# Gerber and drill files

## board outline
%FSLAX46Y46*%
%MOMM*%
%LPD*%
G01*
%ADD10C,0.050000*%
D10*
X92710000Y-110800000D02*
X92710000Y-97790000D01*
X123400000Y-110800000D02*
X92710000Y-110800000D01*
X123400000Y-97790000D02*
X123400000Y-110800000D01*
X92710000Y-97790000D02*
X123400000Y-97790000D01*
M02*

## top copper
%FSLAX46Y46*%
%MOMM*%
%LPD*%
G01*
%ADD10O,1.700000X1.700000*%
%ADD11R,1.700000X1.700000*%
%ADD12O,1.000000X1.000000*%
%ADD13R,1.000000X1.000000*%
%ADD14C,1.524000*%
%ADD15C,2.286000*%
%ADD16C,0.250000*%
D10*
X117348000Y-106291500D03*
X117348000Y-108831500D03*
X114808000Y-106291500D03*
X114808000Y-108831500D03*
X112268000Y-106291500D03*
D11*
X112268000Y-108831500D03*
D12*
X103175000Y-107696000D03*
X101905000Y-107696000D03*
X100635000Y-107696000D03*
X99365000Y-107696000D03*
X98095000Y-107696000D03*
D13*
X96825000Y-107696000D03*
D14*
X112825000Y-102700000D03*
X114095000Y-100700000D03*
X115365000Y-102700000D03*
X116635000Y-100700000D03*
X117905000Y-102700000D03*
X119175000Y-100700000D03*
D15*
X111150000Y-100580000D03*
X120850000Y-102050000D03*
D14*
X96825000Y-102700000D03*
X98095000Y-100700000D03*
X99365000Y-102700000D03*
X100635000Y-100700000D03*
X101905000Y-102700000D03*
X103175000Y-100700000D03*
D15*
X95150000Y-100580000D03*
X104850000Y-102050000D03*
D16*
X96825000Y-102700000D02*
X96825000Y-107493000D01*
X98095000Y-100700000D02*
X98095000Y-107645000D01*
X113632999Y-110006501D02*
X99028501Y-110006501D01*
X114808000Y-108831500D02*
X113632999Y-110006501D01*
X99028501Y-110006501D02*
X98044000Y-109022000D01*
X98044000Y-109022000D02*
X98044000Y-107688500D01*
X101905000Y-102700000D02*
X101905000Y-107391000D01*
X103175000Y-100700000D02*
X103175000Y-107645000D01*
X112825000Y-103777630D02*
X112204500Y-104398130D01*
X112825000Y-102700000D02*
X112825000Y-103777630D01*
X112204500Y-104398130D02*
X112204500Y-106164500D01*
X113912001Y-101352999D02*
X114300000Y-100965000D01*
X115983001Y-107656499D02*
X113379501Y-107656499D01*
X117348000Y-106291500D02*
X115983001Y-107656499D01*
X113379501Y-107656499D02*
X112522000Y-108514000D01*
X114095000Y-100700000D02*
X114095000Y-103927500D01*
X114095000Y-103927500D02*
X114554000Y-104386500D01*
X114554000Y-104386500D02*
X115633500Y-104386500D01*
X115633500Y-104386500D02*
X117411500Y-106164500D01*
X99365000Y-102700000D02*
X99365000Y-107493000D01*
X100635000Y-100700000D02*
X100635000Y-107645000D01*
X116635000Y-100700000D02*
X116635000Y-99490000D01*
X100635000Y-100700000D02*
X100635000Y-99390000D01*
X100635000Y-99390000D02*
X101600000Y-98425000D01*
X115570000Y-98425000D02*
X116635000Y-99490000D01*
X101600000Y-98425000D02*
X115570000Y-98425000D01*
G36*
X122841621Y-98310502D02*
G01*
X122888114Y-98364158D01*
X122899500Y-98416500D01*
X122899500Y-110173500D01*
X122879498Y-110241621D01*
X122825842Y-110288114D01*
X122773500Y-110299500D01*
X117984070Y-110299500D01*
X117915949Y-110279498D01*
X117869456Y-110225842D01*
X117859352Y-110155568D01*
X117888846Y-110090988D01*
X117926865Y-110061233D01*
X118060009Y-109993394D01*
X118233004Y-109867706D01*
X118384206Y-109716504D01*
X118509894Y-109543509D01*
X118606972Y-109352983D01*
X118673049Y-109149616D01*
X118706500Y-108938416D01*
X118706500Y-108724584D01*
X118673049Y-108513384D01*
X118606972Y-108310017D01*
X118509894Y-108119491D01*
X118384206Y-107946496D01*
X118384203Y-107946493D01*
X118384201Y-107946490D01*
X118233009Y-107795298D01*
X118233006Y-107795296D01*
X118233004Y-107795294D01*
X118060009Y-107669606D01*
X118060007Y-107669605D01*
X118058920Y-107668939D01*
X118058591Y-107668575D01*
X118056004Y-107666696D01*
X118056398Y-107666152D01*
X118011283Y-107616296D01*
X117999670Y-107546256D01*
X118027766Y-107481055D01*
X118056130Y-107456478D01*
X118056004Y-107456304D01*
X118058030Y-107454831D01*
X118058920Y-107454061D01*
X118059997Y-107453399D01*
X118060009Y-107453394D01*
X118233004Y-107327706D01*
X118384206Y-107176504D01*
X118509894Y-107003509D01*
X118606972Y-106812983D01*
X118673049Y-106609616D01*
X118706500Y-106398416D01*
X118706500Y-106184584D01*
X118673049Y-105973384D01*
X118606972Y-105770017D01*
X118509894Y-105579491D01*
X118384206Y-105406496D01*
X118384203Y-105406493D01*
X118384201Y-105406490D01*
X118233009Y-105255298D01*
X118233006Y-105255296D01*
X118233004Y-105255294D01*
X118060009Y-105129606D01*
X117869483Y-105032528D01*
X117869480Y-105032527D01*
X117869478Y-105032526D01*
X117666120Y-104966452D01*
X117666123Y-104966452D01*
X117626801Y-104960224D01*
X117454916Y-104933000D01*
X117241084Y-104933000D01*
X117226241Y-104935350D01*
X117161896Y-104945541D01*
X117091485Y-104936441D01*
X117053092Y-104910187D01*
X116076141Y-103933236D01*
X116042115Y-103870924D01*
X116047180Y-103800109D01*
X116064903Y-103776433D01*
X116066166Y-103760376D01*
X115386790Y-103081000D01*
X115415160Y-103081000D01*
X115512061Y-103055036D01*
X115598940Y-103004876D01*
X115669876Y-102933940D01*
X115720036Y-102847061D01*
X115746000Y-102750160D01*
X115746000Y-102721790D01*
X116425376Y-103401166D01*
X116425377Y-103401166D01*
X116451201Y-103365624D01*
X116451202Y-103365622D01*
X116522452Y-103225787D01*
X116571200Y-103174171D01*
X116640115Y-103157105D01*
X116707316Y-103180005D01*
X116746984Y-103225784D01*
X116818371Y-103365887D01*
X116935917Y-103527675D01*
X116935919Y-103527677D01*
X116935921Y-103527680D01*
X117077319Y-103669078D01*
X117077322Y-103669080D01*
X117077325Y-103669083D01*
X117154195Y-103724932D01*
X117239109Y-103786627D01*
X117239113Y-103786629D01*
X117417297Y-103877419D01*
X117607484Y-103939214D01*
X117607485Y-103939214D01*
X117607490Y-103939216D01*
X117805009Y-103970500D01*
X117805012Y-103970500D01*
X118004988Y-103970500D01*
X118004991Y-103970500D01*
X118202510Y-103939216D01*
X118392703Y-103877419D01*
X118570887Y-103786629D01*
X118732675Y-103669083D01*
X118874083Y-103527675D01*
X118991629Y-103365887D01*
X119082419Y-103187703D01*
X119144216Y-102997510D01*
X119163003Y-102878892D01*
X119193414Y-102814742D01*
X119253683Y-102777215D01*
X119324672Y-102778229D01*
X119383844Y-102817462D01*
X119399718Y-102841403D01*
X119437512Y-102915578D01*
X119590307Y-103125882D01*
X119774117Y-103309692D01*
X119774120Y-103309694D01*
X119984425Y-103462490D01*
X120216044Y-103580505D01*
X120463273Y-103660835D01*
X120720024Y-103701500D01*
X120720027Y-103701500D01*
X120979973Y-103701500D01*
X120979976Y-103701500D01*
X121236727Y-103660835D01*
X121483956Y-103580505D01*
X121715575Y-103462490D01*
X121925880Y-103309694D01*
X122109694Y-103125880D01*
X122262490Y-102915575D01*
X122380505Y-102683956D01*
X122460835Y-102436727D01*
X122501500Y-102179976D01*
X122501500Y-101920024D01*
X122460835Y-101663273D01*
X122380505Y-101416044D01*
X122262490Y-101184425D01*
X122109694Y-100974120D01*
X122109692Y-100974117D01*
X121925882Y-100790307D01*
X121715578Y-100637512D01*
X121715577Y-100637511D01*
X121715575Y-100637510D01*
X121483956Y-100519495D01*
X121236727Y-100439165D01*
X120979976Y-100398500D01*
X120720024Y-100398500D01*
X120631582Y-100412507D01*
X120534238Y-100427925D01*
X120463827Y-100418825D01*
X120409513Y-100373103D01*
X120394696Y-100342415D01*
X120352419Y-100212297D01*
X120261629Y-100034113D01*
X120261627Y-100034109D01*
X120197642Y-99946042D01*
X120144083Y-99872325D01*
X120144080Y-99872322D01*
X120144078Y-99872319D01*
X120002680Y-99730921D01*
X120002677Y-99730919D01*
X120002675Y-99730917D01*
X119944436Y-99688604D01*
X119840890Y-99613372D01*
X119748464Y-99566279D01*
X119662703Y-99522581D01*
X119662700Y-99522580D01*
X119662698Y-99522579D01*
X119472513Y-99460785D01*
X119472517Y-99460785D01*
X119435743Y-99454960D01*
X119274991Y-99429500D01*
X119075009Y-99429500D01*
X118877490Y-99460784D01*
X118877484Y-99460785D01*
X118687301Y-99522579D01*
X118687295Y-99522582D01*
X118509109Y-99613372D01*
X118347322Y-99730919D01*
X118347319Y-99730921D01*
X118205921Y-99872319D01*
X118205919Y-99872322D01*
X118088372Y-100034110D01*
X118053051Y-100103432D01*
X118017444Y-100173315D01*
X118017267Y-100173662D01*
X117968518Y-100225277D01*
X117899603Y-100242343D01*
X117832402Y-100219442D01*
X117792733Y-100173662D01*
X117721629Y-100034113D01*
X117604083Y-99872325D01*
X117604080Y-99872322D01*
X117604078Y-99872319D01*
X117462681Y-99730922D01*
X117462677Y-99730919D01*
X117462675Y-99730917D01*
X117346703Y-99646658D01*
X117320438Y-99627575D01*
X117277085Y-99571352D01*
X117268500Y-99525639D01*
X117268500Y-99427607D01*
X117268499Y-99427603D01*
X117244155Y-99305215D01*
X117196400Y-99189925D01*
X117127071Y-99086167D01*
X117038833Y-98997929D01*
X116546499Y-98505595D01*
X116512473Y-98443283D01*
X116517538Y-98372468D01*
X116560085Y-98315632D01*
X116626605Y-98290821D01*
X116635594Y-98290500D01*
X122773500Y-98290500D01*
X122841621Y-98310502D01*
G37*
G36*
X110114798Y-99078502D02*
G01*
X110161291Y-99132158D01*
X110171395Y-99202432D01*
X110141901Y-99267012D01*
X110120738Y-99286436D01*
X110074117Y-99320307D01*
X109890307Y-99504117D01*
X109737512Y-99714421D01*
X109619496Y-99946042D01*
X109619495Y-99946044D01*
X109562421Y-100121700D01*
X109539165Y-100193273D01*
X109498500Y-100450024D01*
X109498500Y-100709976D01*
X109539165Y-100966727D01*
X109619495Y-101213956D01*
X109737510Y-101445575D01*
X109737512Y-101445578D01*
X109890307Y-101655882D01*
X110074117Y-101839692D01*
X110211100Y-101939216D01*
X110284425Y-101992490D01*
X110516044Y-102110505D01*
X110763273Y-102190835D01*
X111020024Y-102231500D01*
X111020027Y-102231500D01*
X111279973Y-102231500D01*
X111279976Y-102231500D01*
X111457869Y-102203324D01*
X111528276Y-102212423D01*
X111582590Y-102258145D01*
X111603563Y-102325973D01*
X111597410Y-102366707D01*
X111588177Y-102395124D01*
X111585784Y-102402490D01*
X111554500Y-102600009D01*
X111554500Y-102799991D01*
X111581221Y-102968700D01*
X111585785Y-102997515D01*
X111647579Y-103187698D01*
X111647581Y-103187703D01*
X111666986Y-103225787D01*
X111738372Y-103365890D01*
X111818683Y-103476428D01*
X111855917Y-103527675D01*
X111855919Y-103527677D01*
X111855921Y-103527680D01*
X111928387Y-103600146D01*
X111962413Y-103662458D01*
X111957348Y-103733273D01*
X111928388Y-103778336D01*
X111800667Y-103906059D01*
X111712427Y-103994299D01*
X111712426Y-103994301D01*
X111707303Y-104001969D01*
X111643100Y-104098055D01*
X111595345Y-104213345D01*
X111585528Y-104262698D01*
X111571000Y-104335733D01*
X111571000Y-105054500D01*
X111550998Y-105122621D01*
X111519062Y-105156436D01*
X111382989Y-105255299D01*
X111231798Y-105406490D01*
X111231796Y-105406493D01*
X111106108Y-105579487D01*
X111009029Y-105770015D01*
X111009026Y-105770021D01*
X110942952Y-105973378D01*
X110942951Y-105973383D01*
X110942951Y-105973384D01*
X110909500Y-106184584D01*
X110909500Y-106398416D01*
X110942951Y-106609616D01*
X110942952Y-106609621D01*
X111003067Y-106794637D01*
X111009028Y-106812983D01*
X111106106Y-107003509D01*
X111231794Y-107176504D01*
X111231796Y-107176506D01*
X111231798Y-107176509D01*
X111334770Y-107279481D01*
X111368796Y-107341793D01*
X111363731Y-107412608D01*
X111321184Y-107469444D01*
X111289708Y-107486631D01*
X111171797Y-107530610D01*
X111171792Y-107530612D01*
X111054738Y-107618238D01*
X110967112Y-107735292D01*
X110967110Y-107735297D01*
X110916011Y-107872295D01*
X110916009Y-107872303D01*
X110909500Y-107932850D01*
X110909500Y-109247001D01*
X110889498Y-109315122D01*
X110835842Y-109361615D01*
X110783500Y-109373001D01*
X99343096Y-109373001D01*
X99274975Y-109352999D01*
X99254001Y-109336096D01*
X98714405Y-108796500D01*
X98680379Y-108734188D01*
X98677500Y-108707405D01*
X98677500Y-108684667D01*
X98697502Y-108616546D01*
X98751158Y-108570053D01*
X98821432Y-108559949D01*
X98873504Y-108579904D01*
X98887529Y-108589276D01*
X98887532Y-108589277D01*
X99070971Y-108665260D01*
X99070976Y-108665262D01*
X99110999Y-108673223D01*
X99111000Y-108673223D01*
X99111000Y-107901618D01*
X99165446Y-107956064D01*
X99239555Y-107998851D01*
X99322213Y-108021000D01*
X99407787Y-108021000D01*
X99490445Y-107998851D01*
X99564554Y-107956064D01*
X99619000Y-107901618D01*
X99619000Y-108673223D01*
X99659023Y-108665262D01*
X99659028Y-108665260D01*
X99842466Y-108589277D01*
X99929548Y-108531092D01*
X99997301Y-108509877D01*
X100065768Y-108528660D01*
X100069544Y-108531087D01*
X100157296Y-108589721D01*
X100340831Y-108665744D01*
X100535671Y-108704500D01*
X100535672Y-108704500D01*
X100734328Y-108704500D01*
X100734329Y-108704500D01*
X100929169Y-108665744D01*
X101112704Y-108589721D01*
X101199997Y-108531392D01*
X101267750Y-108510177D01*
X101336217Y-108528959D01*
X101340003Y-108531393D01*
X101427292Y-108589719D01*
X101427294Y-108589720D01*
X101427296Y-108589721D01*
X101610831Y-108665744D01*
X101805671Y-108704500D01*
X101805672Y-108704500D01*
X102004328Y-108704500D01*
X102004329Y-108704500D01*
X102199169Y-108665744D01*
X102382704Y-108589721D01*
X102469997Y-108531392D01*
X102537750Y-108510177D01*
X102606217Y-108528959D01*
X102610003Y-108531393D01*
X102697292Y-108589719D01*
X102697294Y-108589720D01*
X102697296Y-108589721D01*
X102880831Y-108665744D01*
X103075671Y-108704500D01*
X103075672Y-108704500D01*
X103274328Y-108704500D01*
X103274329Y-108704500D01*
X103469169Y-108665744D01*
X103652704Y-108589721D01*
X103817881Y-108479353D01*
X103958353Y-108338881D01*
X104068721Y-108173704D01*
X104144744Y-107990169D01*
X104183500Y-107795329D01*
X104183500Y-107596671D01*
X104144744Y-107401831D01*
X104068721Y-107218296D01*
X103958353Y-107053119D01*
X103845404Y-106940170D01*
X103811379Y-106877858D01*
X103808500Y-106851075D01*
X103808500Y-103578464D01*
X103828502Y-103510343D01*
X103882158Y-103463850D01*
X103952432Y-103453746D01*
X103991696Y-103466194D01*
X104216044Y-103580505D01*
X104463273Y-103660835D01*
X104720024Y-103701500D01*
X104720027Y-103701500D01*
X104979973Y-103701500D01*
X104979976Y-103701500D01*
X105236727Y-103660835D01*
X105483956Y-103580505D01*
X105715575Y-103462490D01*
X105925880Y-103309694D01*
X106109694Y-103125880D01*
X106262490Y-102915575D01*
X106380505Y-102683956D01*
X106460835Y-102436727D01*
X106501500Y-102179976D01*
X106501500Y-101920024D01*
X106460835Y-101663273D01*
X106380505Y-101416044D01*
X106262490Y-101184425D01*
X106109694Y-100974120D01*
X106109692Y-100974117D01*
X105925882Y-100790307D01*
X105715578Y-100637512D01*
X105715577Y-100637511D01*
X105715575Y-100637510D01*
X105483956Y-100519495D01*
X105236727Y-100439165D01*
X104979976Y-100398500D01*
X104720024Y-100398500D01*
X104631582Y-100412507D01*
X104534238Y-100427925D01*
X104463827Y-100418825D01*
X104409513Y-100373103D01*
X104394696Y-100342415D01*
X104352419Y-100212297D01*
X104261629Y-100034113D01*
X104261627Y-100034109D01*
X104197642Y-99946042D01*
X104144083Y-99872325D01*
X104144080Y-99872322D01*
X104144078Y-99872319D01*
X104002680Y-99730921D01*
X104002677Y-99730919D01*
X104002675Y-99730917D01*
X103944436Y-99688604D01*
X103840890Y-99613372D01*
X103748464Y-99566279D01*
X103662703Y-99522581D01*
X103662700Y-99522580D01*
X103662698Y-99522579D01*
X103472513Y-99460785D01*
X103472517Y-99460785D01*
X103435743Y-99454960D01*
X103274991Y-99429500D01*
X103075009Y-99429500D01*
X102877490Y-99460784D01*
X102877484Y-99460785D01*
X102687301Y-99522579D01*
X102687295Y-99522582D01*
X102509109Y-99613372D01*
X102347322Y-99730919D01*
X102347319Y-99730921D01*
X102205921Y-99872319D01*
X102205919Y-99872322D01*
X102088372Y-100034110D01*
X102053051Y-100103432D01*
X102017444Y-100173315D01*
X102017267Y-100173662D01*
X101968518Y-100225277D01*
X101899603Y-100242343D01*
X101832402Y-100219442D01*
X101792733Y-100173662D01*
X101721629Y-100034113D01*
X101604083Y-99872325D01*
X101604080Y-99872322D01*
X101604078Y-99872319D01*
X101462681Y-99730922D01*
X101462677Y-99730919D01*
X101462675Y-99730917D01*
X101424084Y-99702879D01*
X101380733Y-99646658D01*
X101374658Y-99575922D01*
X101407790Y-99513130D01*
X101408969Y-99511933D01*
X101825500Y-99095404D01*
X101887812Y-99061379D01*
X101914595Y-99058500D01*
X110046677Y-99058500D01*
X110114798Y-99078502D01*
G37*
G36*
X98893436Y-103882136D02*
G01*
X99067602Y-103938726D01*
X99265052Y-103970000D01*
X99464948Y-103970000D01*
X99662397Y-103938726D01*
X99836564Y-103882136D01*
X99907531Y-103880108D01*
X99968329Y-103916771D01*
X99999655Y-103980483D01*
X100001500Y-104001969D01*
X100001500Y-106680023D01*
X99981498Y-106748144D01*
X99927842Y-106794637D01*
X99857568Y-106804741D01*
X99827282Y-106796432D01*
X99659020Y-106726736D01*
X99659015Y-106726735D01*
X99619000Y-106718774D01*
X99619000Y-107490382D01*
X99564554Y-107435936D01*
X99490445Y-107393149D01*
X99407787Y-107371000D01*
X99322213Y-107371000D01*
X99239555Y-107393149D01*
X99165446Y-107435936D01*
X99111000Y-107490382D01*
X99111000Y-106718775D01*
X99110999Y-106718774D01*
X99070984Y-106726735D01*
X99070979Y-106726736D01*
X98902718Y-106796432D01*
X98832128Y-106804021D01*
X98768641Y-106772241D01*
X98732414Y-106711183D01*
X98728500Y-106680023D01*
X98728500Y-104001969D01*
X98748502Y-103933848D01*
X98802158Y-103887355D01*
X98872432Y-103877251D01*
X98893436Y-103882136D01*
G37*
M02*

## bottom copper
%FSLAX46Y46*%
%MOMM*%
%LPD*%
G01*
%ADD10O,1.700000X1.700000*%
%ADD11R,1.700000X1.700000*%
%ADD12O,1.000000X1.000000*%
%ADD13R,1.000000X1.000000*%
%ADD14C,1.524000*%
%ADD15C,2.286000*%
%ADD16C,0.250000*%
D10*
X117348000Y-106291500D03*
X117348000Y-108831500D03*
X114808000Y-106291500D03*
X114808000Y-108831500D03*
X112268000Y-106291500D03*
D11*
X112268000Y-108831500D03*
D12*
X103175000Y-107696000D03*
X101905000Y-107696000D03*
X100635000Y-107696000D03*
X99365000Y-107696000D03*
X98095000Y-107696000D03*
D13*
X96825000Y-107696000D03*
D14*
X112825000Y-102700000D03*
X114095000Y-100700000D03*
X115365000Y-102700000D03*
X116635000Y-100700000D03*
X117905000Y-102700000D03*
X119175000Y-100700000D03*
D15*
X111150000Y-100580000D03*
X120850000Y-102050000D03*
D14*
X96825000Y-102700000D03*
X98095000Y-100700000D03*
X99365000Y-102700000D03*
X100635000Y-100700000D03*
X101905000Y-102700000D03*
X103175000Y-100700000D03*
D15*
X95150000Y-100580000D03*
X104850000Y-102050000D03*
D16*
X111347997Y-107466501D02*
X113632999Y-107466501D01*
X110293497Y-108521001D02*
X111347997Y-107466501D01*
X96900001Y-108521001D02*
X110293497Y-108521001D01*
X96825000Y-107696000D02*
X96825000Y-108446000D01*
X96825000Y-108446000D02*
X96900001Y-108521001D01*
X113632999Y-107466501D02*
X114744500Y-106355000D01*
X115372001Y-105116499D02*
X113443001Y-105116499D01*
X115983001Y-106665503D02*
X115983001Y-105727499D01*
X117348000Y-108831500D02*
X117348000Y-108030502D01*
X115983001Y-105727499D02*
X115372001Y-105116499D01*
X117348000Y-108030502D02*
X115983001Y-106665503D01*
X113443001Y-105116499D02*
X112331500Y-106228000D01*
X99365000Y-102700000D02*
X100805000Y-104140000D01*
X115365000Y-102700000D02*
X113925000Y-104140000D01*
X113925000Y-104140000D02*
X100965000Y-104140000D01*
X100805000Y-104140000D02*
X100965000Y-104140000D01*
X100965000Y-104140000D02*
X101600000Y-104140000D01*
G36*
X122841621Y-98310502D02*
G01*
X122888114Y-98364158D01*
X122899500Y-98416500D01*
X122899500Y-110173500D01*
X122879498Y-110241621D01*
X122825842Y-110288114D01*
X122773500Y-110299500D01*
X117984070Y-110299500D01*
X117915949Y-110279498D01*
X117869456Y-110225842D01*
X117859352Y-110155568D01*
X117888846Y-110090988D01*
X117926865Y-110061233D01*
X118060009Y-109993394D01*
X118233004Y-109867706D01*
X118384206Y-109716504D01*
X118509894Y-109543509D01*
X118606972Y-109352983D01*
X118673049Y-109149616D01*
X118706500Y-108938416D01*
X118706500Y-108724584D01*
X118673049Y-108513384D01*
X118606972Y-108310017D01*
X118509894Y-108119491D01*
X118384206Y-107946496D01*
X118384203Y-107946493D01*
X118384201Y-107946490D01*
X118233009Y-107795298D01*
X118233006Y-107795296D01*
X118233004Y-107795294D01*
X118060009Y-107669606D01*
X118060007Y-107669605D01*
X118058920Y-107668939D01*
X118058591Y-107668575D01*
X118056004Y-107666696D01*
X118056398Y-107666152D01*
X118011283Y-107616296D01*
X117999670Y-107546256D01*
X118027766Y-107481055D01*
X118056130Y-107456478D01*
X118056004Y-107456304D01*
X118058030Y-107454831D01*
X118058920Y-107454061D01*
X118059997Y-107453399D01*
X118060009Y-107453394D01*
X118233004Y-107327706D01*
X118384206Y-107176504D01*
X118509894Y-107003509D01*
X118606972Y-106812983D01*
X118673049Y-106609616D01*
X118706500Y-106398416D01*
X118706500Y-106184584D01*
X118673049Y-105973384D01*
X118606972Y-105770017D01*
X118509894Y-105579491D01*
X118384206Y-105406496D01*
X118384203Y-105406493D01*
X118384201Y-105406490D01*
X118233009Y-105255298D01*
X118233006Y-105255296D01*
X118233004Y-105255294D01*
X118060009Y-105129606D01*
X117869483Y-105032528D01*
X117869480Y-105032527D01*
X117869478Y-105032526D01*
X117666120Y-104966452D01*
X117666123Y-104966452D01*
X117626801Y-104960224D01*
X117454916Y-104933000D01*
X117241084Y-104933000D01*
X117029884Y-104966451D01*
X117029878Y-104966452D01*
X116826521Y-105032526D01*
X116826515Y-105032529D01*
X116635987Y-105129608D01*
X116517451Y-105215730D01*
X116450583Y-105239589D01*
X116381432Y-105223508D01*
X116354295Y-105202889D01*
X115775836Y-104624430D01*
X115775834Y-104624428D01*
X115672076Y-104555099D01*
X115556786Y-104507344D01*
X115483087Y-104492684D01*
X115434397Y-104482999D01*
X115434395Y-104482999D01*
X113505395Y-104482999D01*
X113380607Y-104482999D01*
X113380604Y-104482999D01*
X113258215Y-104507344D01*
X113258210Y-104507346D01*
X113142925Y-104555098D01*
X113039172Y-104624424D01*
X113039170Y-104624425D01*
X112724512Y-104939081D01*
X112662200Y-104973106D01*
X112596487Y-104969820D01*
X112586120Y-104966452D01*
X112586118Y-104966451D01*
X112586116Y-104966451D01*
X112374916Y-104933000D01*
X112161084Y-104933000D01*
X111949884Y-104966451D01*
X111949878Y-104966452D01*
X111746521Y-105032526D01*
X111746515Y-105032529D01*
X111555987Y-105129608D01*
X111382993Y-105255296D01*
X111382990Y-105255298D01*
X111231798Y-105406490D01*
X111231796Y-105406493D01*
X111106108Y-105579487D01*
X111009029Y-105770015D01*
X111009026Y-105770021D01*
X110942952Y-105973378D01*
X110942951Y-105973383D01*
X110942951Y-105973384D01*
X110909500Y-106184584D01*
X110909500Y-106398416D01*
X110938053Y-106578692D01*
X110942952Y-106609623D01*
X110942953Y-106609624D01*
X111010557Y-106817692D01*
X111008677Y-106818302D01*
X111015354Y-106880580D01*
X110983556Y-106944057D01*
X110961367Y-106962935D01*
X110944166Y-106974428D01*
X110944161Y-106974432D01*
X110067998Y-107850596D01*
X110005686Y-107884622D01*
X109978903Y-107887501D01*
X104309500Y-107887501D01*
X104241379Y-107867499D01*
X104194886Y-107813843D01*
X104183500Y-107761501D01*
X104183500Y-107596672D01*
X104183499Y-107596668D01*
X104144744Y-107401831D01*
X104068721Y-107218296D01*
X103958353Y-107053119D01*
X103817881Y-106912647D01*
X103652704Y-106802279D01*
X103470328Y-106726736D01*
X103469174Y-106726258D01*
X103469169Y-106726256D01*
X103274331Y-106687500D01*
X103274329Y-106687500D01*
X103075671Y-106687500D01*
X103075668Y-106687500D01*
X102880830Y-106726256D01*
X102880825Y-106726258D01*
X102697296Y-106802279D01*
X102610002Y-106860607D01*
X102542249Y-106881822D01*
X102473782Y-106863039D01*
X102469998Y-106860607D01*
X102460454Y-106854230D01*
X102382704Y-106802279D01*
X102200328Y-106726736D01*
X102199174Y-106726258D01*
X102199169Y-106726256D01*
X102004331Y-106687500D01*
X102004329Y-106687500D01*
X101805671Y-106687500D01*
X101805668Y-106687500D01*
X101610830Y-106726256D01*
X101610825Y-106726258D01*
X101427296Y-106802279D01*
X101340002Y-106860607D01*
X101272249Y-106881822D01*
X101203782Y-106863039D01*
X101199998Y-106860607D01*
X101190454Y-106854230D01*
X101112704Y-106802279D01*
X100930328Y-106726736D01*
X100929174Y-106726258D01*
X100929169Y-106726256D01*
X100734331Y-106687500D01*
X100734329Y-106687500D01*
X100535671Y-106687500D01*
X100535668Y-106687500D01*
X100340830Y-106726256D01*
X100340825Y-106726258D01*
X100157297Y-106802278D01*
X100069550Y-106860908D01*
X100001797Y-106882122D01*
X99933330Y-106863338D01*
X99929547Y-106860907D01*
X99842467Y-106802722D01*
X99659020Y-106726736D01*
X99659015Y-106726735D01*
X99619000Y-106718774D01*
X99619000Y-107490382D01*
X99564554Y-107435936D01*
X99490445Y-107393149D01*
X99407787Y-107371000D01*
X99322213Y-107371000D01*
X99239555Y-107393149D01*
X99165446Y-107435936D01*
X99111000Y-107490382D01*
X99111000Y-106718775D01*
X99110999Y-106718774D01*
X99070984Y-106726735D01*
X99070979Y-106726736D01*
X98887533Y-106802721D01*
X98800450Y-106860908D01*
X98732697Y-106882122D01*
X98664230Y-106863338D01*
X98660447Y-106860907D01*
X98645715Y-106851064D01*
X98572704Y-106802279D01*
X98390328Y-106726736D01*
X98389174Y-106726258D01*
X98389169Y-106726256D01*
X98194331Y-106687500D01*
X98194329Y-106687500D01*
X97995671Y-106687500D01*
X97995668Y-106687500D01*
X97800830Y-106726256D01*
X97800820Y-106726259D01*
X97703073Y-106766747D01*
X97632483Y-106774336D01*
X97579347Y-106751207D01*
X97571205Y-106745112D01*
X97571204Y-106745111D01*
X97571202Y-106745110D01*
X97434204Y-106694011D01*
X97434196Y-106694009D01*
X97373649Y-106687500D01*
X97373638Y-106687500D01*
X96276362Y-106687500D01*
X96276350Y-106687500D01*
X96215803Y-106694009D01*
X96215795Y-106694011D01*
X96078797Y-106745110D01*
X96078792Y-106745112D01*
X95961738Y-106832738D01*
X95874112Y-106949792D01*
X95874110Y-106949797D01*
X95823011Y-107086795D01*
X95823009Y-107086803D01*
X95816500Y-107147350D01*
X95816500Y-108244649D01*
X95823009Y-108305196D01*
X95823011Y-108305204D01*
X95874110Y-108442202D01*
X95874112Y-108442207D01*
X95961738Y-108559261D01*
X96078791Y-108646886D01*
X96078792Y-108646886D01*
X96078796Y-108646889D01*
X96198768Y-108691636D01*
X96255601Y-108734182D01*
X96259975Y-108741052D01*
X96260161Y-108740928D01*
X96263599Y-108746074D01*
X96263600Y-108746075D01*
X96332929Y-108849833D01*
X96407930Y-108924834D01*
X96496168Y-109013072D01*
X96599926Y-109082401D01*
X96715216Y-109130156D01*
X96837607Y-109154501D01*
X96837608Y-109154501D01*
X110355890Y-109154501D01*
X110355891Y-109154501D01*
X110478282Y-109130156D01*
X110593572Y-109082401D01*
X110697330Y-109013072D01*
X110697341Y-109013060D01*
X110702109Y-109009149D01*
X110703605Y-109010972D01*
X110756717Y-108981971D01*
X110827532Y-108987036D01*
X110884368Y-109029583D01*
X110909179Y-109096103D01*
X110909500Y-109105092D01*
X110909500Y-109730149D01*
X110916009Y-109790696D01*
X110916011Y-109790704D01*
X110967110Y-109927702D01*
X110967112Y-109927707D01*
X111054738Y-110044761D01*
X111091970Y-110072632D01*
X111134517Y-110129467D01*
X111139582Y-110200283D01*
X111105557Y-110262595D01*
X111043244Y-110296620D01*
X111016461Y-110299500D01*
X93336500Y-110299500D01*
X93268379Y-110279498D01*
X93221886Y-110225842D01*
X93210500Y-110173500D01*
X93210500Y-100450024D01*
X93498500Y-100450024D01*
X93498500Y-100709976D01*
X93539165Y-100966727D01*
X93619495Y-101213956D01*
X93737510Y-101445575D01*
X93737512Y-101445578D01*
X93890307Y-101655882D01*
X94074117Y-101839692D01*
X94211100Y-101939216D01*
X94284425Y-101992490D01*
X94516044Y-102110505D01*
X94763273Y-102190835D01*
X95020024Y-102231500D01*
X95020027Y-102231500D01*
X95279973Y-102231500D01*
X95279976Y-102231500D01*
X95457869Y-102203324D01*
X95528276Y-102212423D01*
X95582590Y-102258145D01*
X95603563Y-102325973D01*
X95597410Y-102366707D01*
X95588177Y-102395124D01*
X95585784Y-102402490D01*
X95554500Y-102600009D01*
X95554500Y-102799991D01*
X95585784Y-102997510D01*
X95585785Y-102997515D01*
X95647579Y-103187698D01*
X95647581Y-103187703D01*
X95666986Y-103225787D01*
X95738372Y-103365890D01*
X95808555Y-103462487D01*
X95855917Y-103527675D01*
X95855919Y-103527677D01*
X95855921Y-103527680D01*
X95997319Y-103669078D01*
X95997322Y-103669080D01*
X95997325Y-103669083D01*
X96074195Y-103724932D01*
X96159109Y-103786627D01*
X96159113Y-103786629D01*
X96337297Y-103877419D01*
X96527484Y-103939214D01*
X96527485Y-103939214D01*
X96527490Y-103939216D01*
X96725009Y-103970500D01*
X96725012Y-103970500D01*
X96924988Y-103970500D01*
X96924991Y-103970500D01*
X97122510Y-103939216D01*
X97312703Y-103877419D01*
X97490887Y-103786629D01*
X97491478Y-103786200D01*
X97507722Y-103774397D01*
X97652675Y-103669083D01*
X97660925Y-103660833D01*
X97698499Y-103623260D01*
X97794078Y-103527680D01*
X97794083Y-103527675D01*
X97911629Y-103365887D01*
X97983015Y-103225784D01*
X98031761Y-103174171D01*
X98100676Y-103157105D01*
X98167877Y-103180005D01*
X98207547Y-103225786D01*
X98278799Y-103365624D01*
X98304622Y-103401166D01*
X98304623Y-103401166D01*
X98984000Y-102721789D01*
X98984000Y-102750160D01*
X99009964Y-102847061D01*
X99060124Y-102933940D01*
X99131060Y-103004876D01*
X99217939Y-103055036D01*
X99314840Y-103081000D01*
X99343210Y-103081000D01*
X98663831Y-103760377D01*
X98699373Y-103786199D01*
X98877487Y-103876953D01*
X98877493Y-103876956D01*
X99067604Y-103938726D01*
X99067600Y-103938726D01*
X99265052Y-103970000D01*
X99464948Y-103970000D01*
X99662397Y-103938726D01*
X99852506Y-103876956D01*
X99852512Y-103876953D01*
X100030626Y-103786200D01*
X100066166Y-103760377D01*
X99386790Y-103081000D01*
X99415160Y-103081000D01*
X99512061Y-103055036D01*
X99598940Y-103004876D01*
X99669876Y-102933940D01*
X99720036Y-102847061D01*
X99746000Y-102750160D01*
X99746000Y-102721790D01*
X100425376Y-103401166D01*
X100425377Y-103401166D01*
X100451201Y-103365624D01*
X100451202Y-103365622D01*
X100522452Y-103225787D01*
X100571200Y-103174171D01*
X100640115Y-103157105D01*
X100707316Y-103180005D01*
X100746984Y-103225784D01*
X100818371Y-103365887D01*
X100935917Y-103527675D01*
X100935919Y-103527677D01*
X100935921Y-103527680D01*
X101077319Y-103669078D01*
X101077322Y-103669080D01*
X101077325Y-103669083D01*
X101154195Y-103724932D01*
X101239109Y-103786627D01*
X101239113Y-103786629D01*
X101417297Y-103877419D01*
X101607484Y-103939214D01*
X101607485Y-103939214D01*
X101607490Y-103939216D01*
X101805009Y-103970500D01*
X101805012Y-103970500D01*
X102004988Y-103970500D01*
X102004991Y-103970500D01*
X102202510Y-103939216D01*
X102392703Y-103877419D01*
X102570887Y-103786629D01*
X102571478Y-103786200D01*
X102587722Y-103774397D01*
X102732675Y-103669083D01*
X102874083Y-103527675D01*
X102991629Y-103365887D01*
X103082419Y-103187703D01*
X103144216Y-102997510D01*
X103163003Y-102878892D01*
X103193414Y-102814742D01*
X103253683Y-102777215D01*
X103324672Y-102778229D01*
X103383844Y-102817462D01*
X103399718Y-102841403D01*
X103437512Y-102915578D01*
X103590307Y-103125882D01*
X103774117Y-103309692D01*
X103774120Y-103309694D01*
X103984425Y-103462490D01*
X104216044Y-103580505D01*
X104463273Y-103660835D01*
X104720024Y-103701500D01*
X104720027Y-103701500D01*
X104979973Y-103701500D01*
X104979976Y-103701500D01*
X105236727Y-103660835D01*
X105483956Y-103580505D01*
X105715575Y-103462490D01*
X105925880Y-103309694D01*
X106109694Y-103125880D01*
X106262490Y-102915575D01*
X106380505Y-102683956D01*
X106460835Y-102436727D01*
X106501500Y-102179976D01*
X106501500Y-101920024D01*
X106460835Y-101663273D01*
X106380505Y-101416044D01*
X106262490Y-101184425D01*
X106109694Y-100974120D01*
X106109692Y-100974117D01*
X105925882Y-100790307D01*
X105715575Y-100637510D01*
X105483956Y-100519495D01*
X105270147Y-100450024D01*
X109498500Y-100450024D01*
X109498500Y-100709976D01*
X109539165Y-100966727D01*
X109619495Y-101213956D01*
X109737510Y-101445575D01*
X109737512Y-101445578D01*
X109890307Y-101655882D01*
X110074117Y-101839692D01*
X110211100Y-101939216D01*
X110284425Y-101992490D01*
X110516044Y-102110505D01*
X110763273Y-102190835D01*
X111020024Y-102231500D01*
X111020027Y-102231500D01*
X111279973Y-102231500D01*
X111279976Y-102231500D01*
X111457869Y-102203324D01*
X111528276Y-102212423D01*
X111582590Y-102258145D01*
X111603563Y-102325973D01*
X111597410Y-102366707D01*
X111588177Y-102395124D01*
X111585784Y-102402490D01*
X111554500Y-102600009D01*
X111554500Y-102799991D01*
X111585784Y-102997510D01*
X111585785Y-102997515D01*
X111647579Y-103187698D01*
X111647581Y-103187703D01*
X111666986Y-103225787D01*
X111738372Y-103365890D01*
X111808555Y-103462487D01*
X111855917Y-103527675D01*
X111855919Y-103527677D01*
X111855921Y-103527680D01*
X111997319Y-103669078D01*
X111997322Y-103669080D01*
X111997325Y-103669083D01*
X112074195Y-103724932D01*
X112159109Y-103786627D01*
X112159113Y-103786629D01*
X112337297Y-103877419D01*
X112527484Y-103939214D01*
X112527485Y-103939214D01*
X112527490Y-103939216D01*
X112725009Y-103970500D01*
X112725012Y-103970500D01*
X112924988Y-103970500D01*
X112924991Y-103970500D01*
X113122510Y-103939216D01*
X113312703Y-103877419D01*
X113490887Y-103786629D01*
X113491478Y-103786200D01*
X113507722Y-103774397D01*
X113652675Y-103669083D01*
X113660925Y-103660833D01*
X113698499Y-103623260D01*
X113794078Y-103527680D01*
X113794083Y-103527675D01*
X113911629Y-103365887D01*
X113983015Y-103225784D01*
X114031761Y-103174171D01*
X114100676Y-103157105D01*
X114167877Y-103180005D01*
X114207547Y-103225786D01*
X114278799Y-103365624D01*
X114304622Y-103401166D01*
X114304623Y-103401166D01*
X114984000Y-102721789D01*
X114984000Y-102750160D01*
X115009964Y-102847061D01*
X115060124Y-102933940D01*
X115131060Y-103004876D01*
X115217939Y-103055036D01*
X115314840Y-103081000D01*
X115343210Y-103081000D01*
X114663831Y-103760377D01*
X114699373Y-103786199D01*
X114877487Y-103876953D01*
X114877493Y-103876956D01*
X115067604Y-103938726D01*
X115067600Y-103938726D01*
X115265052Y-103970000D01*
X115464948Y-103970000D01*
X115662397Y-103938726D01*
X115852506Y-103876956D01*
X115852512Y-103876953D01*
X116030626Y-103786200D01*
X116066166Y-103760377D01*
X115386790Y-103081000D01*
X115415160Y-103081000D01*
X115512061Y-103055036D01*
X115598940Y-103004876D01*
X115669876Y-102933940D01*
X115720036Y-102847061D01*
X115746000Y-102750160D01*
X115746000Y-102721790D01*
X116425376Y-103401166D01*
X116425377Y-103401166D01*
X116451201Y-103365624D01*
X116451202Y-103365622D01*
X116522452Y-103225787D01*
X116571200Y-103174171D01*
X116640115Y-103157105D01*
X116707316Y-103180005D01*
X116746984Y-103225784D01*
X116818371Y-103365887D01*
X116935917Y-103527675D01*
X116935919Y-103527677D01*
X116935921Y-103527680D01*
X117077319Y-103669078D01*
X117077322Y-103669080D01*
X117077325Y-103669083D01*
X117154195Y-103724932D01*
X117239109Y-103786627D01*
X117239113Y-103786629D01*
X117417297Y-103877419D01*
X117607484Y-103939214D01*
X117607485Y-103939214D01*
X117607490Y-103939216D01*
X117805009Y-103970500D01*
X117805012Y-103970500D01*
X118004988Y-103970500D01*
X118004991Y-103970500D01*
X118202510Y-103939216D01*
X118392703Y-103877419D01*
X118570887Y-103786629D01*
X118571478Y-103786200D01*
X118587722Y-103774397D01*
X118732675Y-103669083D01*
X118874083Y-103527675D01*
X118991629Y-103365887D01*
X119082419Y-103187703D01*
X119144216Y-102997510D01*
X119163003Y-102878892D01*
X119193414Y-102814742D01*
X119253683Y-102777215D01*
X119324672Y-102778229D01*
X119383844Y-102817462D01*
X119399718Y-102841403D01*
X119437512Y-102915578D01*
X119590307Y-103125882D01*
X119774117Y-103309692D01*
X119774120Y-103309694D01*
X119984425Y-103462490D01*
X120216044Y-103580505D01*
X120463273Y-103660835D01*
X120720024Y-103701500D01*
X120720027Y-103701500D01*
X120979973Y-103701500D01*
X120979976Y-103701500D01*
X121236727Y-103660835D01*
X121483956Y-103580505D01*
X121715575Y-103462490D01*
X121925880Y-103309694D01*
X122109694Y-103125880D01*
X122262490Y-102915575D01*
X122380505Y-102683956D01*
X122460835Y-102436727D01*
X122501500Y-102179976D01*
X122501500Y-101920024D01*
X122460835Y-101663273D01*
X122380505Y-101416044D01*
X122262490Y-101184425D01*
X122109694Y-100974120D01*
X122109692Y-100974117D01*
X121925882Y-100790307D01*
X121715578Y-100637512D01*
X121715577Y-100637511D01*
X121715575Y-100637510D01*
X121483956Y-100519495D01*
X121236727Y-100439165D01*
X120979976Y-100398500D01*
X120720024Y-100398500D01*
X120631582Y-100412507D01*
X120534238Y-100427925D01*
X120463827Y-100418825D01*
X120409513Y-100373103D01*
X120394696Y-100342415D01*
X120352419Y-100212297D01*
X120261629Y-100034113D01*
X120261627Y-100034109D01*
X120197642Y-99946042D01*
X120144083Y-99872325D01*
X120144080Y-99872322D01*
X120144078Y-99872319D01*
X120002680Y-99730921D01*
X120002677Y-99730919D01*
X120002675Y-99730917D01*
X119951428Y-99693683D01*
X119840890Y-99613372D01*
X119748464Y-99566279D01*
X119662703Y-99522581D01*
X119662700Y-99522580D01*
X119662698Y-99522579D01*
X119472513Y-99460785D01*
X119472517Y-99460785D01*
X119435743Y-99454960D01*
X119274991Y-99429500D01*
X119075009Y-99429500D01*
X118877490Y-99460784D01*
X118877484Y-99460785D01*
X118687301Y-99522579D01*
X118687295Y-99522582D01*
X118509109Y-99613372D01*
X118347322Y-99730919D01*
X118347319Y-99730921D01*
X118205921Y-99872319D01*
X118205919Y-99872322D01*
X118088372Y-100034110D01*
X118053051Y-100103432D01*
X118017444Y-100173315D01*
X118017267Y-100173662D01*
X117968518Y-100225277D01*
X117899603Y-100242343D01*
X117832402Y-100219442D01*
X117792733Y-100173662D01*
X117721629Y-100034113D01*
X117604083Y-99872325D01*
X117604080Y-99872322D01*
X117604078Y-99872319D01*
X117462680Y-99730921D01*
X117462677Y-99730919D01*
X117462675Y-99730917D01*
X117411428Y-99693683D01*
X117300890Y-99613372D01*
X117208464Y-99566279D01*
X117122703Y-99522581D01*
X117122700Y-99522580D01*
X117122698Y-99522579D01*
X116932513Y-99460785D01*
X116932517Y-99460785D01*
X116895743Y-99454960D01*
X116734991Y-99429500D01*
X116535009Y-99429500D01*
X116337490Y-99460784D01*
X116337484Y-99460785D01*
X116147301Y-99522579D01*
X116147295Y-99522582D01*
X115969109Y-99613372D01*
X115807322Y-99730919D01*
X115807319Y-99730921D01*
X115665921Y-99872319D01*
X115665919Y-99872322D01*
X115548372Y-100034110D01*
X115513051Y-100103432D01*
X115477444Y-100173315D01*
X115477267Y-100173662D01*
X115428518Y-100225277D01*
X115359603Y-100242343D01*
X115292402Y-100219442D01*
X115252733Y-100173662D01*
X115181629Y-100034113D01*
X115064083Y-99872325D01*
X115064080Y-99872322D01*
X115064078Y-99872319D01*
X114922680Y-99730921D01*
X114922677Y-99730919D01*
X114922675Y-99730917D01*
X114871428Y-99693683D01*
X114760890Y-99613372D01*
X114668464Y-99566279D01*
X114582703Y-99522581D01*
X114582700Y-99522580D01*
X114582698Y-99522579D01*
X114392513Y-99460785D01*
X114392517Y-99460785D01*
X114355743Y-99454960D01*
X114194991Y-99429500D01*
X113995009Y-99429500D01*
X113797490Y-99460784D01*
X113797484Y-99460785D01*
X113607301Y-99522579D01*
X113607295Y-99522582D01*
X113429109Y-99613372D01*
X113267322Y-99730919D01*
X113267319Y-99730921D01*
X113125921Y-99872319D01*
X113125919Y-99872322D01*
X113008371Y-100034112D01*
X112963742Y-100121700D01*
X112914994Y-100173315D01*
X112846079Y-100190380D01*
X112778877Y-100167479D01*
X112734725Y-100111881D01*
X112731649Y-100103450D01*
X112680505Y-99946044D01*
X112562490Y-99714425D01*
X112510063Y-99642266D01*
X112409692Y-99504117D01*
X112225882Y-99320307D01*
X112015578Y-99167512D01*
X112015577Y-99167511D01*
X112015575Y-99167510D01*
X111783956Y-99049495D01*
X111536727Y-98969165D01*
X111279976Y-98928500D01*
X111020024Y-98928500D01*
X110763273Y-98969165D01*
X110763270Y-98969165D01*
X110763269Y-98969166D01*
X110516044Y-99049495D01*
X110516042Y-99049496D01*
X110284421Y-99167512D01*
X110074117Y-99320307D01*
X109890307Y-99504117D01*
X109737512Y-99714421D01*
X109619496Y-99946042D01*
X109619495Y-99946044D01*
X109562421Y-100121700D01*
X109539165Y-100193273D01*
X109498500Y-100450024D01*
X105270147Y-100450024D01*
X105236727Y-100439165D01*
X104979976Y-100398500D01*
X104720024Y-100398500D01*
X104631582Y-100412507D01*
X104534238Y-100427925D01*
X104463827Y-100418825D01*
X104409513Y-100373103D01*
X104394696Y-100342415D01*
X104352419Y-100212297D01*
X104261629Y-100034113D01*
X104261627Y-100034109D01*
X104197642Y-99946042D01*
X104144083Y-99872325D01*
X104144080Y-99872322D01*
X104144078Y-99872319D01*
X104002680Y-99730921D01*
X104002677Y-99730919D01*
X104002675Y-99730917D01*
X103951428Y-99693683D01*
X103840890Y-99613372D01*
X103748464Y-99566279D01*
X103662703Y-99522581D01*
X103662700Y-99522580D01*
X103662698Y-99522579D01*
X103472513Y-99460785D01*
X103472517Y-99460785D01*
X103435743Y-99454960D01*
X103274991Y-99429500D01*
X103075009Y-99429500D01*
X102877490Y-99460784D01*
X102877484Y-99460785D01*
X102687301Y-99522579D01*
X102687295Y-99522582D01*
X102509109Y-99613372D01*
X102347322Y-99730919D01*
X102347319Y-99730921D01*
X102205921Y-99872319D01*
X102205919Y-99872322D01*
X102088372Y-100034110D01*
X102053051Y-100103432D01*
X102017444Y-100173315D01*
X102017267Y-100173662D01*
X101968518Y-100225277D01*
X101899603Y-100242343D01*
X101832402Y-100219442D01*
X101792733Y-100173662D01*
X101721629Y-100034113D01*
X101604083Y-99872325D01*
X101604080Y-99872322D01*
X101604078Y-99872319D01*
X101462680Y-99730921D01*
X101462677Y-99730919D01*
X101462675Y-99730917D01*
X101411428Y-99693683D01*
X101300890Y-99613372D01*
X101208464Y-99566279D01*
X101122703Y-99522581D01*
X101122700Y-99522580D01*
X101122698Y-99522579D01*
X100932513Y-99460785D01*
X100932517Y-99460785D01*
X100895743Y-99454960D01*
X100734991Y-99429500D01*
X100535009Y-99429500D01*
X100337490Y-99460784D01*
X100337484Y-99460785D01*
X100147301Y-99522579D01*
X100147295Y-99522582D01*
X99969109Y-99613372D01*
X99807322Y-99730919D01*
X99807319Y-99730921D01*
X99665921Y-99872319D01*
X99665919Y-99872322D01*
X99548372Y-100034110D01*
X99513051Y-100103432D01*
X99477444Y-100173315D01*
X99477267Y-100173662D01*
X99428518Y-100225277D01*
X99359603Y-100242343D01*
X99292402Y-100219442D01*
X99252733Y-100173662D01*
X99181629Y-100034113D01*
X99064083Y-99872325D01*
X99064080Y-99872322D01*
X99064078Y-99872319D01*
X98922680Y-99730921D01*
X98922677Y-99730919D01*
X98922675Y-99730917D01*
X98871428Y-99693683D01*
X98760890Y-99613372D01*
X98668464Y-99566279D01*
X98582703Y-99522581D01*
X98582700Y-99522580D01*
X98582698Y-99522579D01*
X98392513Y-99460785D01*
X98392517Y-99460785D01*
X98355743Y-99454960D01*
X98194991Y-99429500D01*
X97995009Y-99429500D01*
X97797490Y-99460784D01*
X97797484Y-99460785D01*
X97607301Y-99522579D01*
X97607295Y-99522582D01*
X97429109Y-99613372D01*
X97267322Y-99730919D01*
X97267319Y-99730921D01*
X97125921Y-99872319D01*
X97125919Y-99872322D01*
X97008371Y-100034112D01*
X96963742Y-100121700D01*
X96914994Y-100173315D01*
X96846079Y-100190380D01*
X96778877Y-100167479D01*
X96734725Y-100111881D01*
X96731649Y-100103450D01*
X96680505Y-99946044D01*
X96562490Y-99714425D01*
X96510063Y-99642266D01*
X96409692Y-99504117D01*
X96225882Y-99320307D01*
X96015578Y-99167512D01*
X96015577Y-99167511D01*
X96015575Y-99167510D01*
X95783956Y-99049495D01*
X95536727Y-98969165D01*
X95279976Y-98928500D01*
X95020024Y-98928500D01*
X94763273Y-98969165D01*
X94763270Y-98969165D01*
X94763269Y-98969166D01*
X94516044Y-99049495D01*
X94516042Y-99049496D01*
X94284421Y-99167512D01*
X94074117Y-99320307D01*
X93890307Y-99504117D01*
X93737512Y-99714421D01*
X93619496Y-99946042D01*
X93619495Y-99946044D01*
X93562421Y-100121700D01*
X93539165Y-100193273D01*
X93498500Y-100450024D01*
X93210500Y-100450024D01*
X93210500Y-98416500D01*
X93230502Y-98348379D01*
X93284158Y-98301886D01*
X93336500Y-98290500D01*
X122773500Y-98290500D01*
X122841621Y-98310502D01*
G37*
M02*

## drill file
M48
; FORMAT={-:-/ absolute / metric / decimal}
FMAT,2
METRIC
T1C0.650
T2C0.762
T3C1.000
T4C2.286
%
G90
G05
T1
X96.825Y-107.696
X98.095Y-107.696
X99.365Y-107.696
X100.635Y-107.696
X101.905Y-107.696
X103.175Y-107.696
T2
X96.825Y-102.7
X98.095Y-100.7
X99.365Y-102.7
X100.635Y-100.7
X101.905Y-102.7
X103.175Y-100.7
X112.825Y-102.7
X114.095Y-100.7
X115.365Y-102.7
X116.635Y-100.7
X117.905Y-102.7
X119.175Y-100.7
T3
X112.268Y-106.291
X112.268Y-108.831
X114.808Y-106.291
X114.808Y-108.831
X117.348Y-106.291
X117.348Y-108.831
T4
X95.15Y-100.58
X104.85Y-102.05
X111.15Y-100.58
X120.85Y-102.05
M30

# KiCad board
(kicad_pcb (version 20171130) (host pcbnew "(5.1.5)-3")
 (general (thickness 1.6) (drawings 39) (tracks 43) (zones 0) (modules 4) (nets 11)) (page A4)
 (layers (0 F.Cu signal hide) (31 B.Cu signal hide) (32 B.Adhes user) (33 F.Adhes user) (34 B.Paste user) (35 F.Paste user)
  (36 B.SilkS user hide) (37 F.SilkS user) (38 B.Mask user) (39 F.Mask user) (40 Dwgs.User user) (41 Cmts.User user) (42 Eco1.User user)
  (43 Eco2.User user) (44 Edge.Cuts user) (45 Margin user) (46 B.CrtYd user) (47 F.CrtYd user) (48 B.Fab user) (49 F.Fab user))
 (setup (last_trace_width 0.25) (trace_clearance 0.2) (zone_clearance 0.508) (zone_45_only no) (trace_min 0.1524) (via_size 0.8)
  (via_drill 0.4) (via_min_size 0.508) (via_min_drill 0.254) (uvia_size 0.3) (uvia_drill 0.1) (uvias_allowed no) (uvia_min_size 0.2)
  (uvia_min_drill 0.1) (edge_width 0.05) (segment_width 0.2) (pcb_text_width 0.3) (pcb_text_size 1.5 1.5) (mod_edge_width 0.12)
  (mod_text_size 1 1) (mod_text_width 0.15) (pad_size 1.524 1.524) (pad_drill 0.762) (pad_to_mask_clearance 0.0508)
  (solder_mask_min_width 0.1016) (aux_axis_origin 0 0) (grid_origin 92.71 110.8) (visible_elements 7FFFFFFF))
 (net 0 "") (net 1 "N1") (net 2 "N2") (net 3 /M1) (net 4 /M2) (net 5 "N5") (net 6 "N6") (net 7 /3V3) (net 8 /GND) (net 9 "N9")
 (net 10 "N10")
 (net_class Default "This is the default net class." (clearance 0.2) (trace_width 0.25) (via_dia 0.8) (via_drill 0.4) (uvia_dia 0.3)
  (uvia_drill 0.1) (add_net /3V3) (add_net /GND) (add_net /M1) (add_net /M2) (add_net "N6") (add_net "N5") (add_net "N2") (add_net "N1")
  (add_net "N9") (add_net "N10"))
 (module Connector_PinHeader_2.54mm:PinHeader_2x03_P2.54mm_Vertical (layer F.Cu) (at 112.268 108.8315 90)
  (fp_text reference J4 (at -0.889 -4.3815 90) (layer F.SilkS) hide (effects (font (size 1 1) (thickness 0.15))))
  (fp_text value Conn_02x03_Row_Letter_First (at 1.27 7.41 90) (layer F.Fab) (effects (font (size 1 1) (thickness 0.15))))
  (pad 6 thru_hole oval (at 2.54 5.08 90) (size 1.7 1.7) (drill 1) (layers *.Cu *.Mask) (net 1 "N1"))
  (pad 5 thru_hole oval (at 0 5.08 90) (size 1.7 1.7) (drill 1) (layers *.Cu *.Mask) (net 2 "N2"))
  (pad 4 thru_hole oval (at 2.54 2.54 90) (size 1.7 1.7) (drill 1) (layers *.Cu *.Mask) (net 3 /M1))
  (pad 3 thru_hole oval (at 0 2.54 90) (size 1.7 1.7) (drill 1) (layers *.Cu *.Mask) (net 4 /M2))
  (pad 2 thru_hole oval (at 2.54 0 90) (size 1.7 1.7) (drill 1) (layers *.Cu *.Mask) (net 2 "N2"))
  (pad 1 thru_hole rect (at 0 0 90) (size 1.7 1.7) (drill 1) (layers *.Cu *.Mask) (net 1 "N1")))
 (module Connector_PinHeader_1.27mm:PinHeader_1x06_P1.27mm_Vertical (layer F.Cu) (at 96.825 107.696 90)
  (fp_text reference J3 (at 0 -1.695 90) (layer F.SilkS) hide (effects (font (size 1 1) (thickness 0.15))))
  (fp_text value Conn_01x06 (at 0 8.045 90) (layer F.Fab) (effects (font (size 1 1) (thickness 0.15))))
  (pad 6 thru_hole oval (at 0 6.35 90) (size 1 1) (drill 0.65) (layers *.Cu *.Mask) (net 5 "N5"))
  (pad 5 thru_hole oval (at 0 5.08 90) (size 1 1) (drill 0.65) (layers *.Cu *.Mask) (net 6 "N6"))
  (pad 4 thru_hole oval (at 0 3.81 90) (size 1 1) (drill 0.65) (layers *.Cu *.Mask) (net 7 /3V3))
  (pad 3 thru_hole oval (at 0 2.54 90) (size 1 1) (drill 0.65) (layers *.Cu *.Mask) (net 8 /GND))
  (pad 2 thru_hole oval (at 0 1.27 90) (size 1 1) (drill 0.65) (layers *.Cu *.Mask) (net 4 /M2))
  (pad 1 thru_hole rect (at 0 0 90) (size 1 1) (drill 0.65) (layers *.Cu *.Mask) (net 3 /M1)))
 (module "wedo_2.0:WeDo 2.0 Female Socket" (layer F.Cu) (at 116 100)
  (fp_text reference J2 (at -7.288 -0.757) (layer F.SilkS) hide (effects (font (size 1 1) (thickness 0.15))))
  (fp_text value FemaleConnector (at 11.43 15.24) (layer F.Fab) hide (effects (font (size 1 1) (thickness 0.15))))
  (pad 1 thru_hole circle (at -3.175 2.7) (size 1.524 1.524) (drill 0.762) (layers *.Cu *.Mask) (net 2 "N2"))
  (pad 2 thru_hole circle (at -1.905 0.7) (size 1.524 1.524) (drill 0.762) (layers *.Cu *.Mask) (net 1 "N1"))
  (pad 3 thru_hole circle (at -0.635 2.7) (size 1.524 1.524) (drill 0.762) (layers *.Cu *.Mask) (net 8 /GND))
  (pad 4 thru_hole circle (at 0.635 0.7) (size 1.524 1.524) (drill 0.762) (layers *.Cu *.Mask) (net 7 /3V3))
  (pad 5 thru_hole circle (at 1.905 2.7) (size 1.524 1.524) (drill 0.762) (layers *.Cu *.Mask) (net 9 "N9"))
  (pad 6 thru_hole circle (at 3.175 0.7) (size 1.524 1.524) (drill 0.762) (layers *.Cu *.Mask) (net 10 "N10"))
  (pad "" thru_hole circle (at -4.85 0.58) (size 2.286 2.286) (drill 2.286) (layers *.Cu *.Mask))
  (pad "" thru_hole circle (at 4.85 2.05) (size 2.286 2.286) (drill 2.286) (layers *.Cu *.Mask)))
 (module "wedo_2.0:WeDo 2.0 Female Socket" (layer F.Cu) (at 100 100)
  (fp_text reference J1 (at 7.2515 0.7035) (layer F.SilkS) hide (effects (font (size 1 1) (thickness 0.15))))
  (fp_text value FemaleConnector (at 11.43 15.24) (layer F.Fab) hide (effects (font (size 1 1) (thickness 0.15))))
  (pad 1 thru_hole circle (at -3.175 2.7) (size 1.524 1.524) (drill 0.762) (layers *.Cu *.Mask) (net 3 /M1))
  (pad 2 thru_hole circle (at -1.905 0.7) (size 1.524 1.524) (drill 0.762) (layers *.Cu *.Mask) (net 4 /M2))
  (pad 3 thru_hole circle (at -0.635 2.7) (size 1.524 1.524) (drill 0.762) (layers *.Cu *.Mask) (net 8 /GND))
  (pad 4 thru_hole circle (at 0.635 0.7) (size 1.524 1.524) (drill 0.762) (layers *.Cu *.Mask) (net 7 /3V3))
  (pad 5 thru_hole circle (at 1.905 2.7) (size 1.524 1.524) (drill 0.762) (layers *.Cu *.Mask) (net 6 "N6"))
  (pad 6 thru_hole circle (at 3.175 0.7) (size 1.524 1.524) (drill 0.762) (layers *.Cu *.Mask) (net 5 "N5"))
  (pad "" thru_hole circle (at -4.85 0.58) (size 2.286 2.286) (drill 2.286) (layers *.Cu *.Mask))
  (pad "" thru_hole circle (at 4.85 2.05) (size 2.286 2.286) (drill 2.286) (layers *.Cu *.Mask)))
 (gr_line (start 92.71 110.8) (end 92.71 97.79) (layer Edge.Cuts) (width 0.05))
 (gr_line (start 123.4 110.8) (end 92.71 110.8) (layer Edge.Cuts) (width 0.05))
 (gr_line (start 123.4 97.79) (end 123.4 110.8) (layer Edge.Cuts) (width 0.05))
 (gr_line (start 92.71 97.79) (end 123.4 97.79) (layer Edge.Cuts) (width 0.05))
 (segment (start 96.825 102.7) (end 96.825 107.493) (width 0.25) (layer F.Cu) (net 3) (status 30))
 (segment (start 111.347997 107.466501) (end 113.632999 107.466501) (width 0.25) (layer B.Cu) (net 3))
 (segment (start 110.293497 108.521001) (end 111.347997 107.466501) (width 0.25) (layer B.Cu) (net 3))
 (segment (start 96.900001 108.521001) (end 110.293497 108.521001) (width 0.25) (layer B.Cu) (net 3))
 (segment (start 96.825 107.696) (end 96.825 108.446) (width 0.25) (layer B.Cu) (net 3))
 (segment (start 96.825 108.446) (end 96.900001 108.521001) (width 0.25) (layer B.Cu) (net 3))
 (segment (start 113.632999 107.466501) (end 114.7445 106.355) (width 0.25) (layer B.Cu) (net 3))
 (segment (start 98.095 100.7) (end 98.095 107.645) (width 0.25) (layer F.Cu) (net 4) (status 30))
 (segment (start 113.632999 110.006501) (end 99.028501 110.006501) (width 0.25) (layer F.Cu) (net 4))
 (segment (start 114.808 108.8315) (end 113.632999 110.006501) (width 0.25) (layer F.Cu) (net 4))
 (segment (start 99.028501 110.006501) (end 98.044 109.022) (width 0.25) (layer F.Cu) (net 4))
 (segment (start 98.044 109.022) (end 98.044 107.6885) (width 0.25) (layer F.Cu) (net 4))
 (segment (start 101.905 102.7) (end 101.905 107.391) (width 0.25) (layer F.Cu) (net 6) (status 30))
 (segment (start 103.175 100.7) (end 103.175 107.645) (width 0.25) (layer F.Cu) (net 5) (status 30))
 (segment (start 112.825 103.77763) (end 112.2045 104.39813) (width 0.25) (layer F.Cu) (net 2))
 (segment (start 112.825 102.7) (end 112.825 103.77763) (width 0.25) (layer F.Cu) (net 2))
 (segment (start 112.2045 104.39813) (end 112.2045 106.1645) (width 0.25) (layer F.Cu) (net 2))
 (segment (start 115.372001 105.116499) (end 113.443001 105.116499) (width 0.25) (layer B.Cu) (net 2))
 (segment (start 115.983001 106.665503) (end 115.983001 105.727499) (width 0.25) (layer B.Cu) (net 2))
 (segment (start 117.348 108.8315) (end 117.348 108.030502) (width 0.25) (layer B.Cu) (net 2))
 (segment (start 115.983001 105.727499) (end 115.372001 105.116499) (width 0.25) (layer B.Cu) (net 2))
 (segment (start 117.348 108.030502) (end 115.983001 106.665503) (width 0.25) (layer B.Cu) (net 2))
 (segment (start 113.443001 105.116499) (end 112.3315 106.228) (width 0.25) (layer B.Cu) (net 2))
 (segment (start 113.912001 101.352999) (end 114.3 100.965) (width 0.25) (layer F.Cu) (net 1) (status 30))
 (segment (start 115.983001 107.656499) (end 113.379501 107.656499) (width 0.25) (layer F.Cu) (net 1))
 (segment (start 117.348 106.2915) (end 115.983001 107.656499) (width 0.25) (layer F.Cu) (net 1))
 (segment (start 113.379501 107.656499) (end 112.522 108.514) (width 0.25) (layer F.Cu) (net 1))
 (segment (start 114.095 100.7) (end 114.095 103.9275) (width 0.25) (layer F.Cu) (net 1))
 (segment (start 114.095 103.9275) (end 114.554 104.3865) (width 0.25) (layer F.Cu) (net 1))
 (segment (start 114.554 104.3865) (end 115.6335 104.3865) (width 0.25) (layer F.Cu) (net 1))
 (segment (start 115.6335 104.3865) (end 117.4115 106.1645) (width 0.25) (layer F.Cu) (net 1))
 (segment (start 99.365 102.7) (end 99.365 107.493) (width 0.25) (layer F.Cu) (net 8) (status 30))
 (segment (start 99.365 102.7) (end 100.805 104.14) (width 0.25) (layer B.Cu) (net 8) (status 10))
 (segment (start 115.365 102.7) (end 113.925 104.14) (width 0.25) (layer B.Cu) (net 8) (status 10))
 (segment (start 113.925 104.14) (end 100.965 104.14) (width 0.25) (layer B.Cu) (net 8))
 (segment (start 100.805 104.14) (end 100.965 104.14) (width 0.25) (layer B.Cu) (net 8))
 (segment (start 100.965 104.14) (end 101.6 104.14) (width 0.25) (layer B.Cu) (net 8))
 (segment (start 100.635 100.7) (end 100.635 107.645) (width 0.25) (layer F.Cu) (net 7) (status 30))
 (segment (start 116.635 100.7) (end 116.635 99.49) (width 0.25) (layer F.Cu) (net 7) (status 10))
 (segment (start 100.635 100.7) (end 100.635 99.39) (width 0.25) (layer F.Cu) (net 7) (status 10))
 (segment (start 100.635 99.39) (end 101.6 98.425) (width 0.25) (layer F.Cu) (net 7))
 (segment (start 115.57 98.425) (end 116.635 99.49) (width 0.25) (layer F.Cu) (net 7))
 (segment (start 101.6 98.425) (end 115.57 98.425) (width 0.25) (layer F.Cu) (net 7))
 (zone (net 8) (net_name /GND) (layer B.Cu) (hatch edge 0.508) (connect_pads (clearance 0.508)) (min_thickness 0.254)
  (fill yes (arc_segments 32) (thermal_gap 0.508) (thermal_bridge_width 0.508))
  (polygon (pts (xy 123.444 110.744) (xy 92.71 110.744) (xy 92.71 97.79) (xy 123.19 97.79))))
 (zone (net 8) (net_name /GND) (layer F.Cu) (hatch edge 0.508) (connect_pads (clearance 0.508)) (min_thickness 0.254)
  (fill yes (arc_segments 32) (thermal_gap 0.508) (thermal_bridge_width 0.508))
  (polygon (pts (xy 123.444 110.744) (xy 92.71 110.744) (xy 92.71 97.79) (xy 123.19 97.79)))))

